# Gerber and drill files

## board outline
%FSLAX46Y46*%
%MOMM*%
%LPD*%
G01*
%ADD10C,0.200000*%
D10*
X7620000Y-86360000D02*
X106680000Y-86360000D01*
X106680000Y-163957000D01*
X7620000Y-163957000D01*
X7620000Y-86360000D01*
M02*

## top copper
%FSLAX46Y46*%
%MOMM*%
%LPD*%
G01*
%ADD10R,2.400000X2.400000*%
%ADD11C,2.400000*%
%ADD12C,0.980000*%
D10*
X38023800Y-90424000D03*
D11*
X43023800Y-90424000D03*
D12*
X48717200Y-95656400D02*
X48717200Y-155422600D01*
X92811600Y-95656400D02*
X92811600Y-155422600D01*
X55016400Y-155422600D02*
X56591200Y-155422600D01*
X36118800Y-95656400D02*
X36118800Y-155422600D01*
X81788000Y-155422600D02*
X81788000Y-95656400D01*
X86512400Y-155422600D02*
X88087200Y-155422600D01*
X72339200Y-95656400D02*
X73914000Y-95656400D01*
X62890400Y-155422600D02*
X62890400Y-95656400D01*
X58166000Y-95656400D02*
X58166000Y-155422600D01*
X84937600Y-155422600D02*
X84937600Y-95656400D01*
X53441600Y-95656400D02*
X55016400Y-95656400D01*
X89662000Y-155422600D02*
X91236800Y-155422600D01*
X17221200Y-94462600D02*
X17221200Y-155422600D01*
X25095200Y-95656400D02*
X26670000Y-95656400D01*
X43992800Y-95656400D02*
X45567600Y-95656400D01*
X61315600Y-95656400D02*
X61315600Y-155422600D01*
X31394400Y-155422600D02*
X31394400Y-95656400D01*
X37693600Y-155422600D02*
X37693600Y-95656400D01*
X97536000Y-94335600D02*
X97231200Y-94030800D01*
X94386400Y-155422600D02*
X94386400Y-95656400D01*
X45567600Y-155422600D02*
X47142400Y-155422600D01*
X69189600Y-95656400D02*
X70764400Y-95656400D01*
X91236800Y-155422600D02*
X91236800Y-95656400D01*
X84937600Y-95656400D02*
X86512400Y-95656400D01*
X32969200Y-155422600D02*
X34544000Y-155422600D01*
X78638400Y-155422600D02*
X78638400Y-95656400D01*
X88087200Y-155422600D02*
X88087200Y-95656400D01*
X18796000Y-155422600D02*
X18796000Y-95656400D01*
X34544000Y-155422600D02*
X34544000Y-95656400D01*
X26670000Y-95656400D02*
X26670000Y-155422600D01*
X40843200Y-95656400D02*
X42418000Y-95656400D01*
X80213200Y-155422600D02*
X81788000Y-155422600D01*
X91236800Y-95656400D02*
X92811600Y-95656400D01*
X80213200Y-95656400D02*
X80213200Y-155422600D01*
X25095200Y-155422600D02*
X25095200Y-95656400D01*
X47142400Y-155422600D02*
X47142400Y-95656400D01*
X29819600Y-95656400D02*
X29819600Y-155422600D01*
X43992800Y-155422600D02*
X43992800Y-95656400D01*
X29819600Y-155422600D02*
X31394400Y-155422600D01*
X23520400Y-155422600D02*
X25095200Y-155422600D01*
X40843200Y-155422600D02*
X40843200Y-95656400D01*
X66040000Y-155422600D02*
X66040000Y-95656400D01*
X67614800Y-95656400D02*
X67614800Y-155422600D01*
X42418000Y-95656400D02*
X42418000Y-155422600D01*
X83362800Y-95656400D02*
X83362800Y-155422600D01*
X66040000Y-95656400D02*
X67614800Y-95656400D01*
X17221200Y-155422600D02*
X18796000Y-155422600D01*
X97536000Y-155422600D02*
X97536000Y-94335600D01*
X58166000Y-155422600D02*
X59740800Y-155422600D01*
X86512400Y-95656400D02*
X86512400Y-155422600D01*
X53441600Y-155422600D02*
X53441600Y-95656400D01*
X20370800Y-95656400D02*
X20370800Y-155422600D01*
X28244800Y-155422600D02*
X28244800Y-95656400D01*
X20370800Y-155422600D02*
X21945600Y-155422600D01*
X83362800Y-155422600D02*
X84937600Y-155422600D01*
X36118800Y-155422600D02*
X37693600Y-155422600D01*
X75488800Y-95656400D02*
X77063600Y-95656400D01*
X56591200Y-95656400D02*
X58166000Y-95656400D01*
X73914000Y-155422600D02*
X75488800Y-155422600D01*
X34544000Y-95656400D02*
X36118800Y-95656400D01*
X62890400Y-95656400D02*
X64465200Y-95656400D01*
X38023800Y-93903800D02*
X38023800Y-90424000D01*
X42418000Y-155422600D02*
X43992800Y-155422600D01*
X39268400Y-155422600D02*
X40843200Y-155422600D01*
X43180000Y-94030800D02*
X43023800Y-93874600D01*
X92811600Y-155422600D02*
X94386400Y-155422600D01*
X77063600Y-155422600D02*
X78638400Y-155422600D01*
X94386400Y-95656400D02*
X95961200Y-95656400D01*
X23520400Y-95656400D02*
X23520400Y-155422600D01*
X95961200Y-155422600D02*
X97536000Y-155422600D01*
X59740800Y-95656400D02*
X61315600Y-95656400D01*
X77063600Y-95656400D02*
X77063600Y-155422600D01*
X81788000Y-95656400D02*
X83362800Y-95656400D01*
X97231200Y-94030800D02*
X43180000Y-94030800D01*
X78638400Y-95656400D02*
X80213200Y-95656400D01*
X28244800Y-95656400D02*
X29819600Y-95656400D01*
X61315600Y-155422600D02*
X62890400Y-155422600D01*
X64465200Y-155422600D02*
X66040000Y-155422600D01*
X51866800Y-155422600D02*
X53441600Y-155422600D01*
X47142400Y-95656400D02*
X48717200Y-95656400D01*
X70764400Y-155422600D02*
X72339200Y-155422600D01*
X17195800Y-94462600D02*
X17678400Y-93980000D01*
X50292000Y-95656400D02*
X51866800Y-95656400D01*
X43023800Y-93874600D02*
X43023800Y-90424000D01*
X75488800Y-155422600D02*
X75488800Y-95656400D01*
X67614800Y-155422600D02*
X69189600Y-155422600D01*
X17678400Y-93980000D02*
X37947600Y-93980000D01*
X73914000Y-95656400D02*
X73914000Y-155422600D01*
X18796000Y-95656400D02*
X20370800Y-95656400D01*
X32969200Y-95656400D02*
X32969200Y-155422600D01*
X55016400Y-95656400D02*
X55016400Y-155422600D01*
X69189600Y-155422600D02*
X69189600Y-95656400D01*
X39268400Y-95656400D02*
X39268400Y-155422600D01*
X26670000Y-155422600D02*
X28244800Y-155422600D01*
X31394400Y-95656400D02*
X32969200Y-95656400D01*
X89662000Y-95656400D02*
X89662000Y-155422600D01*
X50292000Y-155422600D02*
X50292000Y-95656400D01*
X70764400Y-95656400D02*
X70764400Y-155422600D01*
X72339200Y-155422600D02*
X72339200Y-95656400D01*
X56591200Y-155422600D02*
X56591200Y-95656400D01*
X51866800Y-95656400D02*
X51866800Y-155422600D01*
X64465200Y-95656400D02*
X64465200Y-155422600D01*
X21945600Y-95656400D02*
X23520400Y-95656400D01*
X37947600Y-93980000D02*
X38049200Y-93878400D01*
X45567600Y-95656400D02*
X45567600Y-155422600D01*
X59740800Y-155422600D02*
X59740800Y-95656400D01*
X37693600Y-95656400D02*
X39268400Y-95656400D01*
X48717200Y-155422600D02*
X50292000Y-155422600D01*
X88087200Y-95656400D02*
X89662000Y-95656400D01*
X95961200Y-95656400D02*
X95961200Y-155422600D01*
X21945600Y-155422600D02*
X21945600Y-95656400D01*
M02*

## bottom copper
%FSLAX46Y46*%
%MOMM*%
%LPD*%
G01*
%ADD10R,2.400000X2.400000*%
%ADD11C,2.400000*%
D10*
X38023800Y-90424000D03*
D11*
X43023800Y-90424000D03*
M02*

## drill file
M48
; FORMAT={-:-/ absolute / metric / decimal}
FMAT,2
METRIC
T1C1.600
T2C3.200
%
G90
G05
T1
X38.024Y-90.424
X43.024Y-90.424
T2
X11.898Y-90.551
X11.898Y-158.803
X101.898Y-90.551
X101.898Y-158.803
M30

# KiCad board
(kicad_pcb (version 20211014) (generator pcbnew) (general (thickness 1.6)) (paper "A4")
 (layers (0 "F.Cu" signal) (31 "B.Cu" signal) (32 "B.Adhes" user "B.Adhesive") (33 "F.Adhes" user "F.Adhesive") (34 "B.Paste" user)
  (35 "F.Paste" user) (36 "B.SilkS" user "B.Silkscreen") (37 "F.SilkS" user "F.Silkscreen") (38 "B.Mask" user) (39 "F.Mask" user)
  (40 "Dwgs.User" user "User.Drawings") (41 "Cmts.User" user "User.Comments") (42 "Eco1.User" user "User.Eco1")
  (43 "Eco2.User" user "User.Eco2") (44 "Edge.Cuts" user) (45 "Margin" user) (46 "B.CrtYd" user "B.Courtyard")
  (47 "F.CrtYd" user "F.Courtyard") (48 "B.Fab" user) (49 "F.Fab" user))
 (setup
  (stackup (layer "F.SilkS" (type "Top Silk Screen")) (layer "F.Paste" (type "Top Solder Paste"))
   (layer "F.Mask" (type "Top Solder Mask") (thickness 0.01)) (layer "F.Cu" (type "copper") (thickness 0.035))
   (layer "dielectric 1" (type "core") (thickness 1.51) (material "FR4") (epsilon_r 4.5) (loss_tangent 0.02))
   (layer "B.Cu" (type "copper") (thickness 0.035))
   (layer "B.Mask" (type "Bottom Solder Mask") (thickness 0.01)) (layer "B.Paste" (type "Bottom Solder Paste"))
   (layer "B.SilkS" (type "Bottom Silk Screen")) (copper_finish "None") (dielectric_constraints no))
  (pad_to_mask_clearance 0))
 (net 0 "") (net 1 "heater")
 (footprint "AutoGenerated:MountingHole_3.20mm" (layer "F.Cu") (at 91.898 142.803)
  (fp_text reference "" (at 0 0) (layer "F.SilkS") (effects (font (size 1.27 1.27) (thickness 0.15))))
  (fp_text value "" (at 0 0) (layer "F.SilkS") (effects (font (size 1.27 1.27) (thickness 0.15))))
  (pad "" np_thru_hole circle (at 10 16) (size 3.2 3.2) (drill 3.2) (layers F&B.Cu *.Mask)))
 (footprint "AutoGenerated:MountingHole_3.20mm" (layer "F.Cu") (at 11.898 90.551)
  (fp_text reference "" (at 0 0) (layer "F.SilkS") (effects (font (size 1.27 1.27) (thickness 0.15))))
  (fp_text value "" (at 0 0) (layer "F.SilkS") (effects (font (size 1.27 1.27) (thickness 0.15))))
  (pad "" np_thru_hole circle locked (at 0 0) (size 3.2 3.2) (drill 3.2) (layers *.Cu *.Mask)))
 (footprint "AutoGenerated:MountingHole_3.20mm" (layer "F.Cu") (at 91.898 90.551)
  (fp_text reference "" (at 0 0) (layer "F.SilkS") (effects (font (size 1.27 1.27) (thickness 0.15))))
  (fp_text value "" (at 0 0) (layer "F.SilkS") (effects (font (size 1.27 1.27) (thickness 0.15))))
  (pad "" np_thru_hole circle (at 10 0) (size 3.2 3.2) (drill 3.2) (layers F&B.Cu *.Mask)))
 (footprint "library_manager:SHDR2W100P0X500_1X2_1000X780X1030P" (layer "F.Cu") (at 38.0238 90.424)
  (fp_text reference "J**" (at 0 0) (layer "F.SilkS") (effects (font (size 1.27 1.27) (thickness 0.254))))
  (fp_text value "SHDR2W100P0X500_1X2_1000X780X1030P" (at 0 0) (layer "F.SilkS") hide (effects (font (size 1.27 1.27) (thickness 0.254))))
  (pad "1" thru_hole rect locked (at 0 0) (size 2.4 2.4) (drill 1.6) (layers *.Cu *.Mask) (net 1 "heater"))
  (pad "2" thru_hole circle locked (at 5 0) (size 2.4 2.4) (drill 1.6) (layers *.Cu *.Mask) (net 1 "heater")))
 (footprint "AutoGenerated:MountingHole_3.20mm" (layer "F.Cu") (at 11.898 142.803)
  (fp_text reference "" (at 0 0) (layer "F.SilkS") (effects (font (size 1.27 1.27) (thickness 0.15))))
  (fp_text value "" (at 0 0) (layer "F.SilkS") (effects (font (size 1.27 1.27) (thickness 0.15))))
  (pad "" np_thru_hole circle (at 0 16) (size 3.2 3.2) (drill 3.2) (layers F&B.Cu *.Mask)))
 (gr_rect (start 7.62 86.36) (end 106.68 163.957) (layer "Edge.Cuts") (width 0.2) (fill none))
 (segment (start 48.7172 95.6564) (end 48.7172 155.4226) (width 0.98) (layer "F.Cu") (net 1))
 (segment (start 92.8116 95.6564) (end 92.8116 155.4226) (width 0.98) (layer "F.Cu") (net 1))
 (segment (start 55.0164 155.4226) (end 56.5912 155.4226) (width 0.98) (layer "F.Cu") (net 1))
 (segment (start 36.1188 95.6564) (end 36.1188 155.4226) (width 0.98) (layer "F.Cu") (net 1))
 (segment (start 81.788 155.4226) (end 81.788 95.6564) (width 0.98) (layer "F.Cu") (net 1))
 (segment (start 86.5124 155.4226) (end 88.0872 155.4226) (width 0.98) (layer "F.Cu") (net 1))
 (segment (start 72.3392 95.6564) (end 73.914 95.6564) (width 0.98) (layer "F.Cu") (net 1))
 (segment (start 62.8904 155.4226) (end 62.8904 95.6564) (width 0.98) (layer "F.Cu") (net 1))
 (segment (start 58.166 95.6564) (end 58.166 155.4226) (width 0.98) (layer "F.Cu") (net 1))
 (segment (start 84.9376 155.4226) (end 84.9376 95.6564) (width 0.98) (layer "F.Cu") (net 1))
 (segment (start 53.4416 95.6564) (end 55.0164 95.6564) (width 0.98) (layer "F.Cu") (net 1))
 (segment (start 89.662 155.4226) (end 91.2368 155.4226) (width 0.98) (layer "F.Cu") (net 1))
 (segment (start 17.2212 94.4626) (end 17.2212 155.4226) (width 0.98) (layer "F.Cu") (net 1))
 (segment (start 25.0952 95.6564) (end 26.67 95.6564) (width 0.98) (layer "F.Cu") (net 1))
 (segment (start 43.9928 95.6564) (end 45.5676 95.6564) (width 0.98) (layer "F.Cu") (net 1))
 (segment (start 61.3156 95.6564) (end 61.3156 155.4226) (width 0.98) (layer "F.Cu") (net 1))
 (segment (start 31.3944 155.4226) (end 31.3944 95.6564) (width 0.98) (layer "F.Cu") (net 1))
 (segment (start 37.6936 155.4226) (end 37.6936 95.6564) (width 0.98) (layer "F.Cu") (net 1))
 (segment (start 97.536 94.3356) (end 97.2312 94.0308) (width 0.98) (layer "F.Cu") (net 1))
 (segment (start 94.3864 155.4226) (end 94.3864 95.6564) (width 0.98) (layer "F.Cu") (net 1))
 (segment (start 45.5676 155.4226) (end 47.1424 155.4226) (width 0.98) (layer "F.Cu") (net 1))
 (segment (start 69.1896 95.6564) (end 70.7644 95.6564) (width 0.98) (layer "F.Cu") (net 1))
 (segment (start 91.2368 155.4226) (end 91.2368 95.6564) (width 0.98) (layer "F.Cu") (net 1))
 (segment (start 84.9376 95.6564) (end 86.5124 95.6564) (width 0.98) (layer "F.Cu") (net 1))
 (segment (start 32.9692 155.4226) (end 34.544 155.4226) (width 0.98) (layer "F.Cu") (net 1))
 (segment (start 78.6384 155.4226) (end 78.6384 95.6564) (width 0.98) (layer "F.Cu") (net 1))
 (segment (start 88.0872 155.4226) (end 88.0872 95.6564) (width 0.98) (layer "F.Cu") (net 1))
 (segment (start 18.796 155.4226) (end 18.796 95.6564) (width 0.98) (layer "F.Cu") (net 1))
 (segment (start 34.544 155.4226) (end 34.544 95.6564) (width 0.98) (layer "F.Cu") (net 1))
 (segment (start 26.67 95.6564) (end 26.67 155.4226) (width 0.98) (layer "F.Cu") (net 1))
 (segment (start 40.8432 95.6564) (end 42.418 95.6564) (width 0.98) (layer "F.Cu") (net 1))
 (segment (start 80.2132 155.4226) (end 81.788 155.4226) (width 0.98) (layer "F.Cu") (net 1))
 (segment (start 91.2368 95.6564) (end 92.8116 95.6564) (width 0.98) (layer "F.Cu") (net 1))
 (segment (start 80.2132 95.6564) (end 80.2132 155.4226) (width 0.98) (layer "F.Cu") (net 1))
 (segment (start 25.0952 155.4226) (end 25.0952 95.6564) (width 0.98) (layer "F.Cu") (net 1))
 (segment (start 47.1424 155.4226) (end 47.1424 95.6564) (width 0.98) (layer "F.Cu") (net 1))
 (segment (start 29.8196 95.6564) (end 29.8196 155.4226) (width 0.98) (layer "F.Cu") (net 1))
 (segment (start 43.9928 155.4226) (end 43.9928 95.6564) (width 0.98) (layer "F.Cu") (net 1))
 (segment (start 29.8196 155.4226) (end 31.3944 155.4226) (width 0.98) (layer "F.Cu") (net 1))
 (segment (start 23.5204 155.4226) (end 25.0952 155.4226) (width 0.98) (layer "F.Cu") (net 1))
 (segment (start 40.8432 155.4226) (end 40.8432 95.6564) (width 0.98) (layer "F.Cu") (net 1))
 (segment (start 66.04 155.4226) (end 66.04 95.6564) (width 0.98) (layer "F.Cu") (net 1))
 (segment (start 67.6148 95.6564) (end 67.6148 155.4226) (width 0.98) (layer "F.Cu") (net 1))
 (segment (start 42.418 95.6564) (end 42.418 155.4226) (width 0.98) (layer "F.Cu") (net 1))
 (segment (start 83.3628 95.6564) (end 83.3628 155.4226) (width 0.98) (layer "F.Cu") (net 1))
 (segment (start 66.04 95.6564) (end 67.6148 95.6564) (width 0.98) (layer "F.Cu") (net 1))
 (segment (start 17.2212 155.4226) (end 18.796 155.4226) (width 0.98) (layer "F.Cu") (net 1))
 (segment (start 97.536 155.4226) (end 97.536 94.3356) (width 0.98) (layer "F.Cu") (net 1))
 (segment (start 58.166 155.4226) (end 59.7408 155.4226) (width 0.98) (layer "F.Cu") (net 1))
 (segment (start 86.5124 95.6564) (end 86.5124 155.4226) (width 0.98) (layer "F.Cu") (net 1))
 (segment (start 53.4416 155.4226) (end 53.4416 95.6564) (width 0.98) (layer "F.Cu") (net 1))
 (segment (start 20.3708 95.6564) (end 20.3708 155.4226) (width 0.98) (layer "F.Cu") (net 1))
 (segment (start 28.2448 155.4226) (end 28.2448 95.6564) (width 0.98) (layer "F.Cu") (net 1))
 (segment (start 20.3708 155.4226) (end 21.9456 155.4226) (width 0.98) (layer "F.Cu") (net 1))
 (segment (start 83.3628 155.4226) (end 84.9376 155.4226) (width 0.98) (layer "F.Cu") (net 1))
 (segment (start 36.1188 155.4226) (end 37.6936 155.4226) (width 0.98) (layer "F.Cu") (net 1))
 (segment (start 75.4888 95.6564) (end 77.0636 95.6564) (width 0.98) (layer "F.Cu") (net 1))
 (segment (start 56.5912 95.6564) (end 58.166 95.6564) (width 0.98) (layer "F.Cu") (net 1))
 (segment (start 73.914 155.4226) (end 75.4888 155.4226) (width 0.98) (layer "F.Cu") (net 1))
 (segment (start 34.544 95.6564) (end 36.1188 95.6564) (width 0.98) (layer "F.Cu") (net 1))
 (segment (start 62.8904 95.6564) (end 64.4652 95.6564) (width 0.98) (layer "F.Cu") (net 1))
 (segment (start 38.0238 93.9038) (end 38.0238 90.424) (width 0.98) (layer "F.Cu") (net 1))
 (segment (start 42.418 155.4226) (end 43.9928 155.4226) (width 0.98) (layer "F.Cu") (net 1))
 (segment (start 39.2684 155.4226) (end 40.8432 155.4226) (width 0.98) (layer "F.Cu") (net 1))
 (segment (start 43.18 94.0308) (end 43.0238 93.8746) (width 0.98) (layer "F.Cu") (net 1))
 (segment (start 92.8116 155.4226) (end 94.3864 155.4226) (width 0.98) (layer "F.Cu") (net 1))
 (segment (start 77.0636 155.4226) (end 78.6384 155.4226) (width 0.98) (layer "F.Cu") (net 1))
 (segment (start 94.3864 95.6564) (end 95.9612 95.6564) (width 0.98) (layer "F.Cu") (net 1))
 (segment (start 23.5204 95.6564) (end 23.5204 155.4226) (width 0.98) (layer "F.Cu") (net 1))
 (segment (start 95.9612 155.4226) (end 97.536 155.4226) (width 0.98) (layer "F.Cu") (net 1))
 (segment (start 59.7408 95.6564) (end 61.3156 95.6564) (width 0.98) (layer "F.Cu") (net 1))
 (segment (start 77.0636 95.6564) (end 77.0636 155.4226) (width 0.98) (layer "F.Cu") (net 1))
 (segment (start 81.788 95.6564) (end 83.3628 95.6564) (width 0.98) (layer "F.Cu") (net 1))
 (segment (start 97.2312 94.0308) (end 43.18 94.0308) (width 0.98) (layer "F.Cu") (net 1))
 (segment (start 78.6384 95.6564) (end 80.2132 95.6564) (width 0.98) (layer "F.Cu") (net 1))
 (segment (start 28.2448 95.6564) (end 29.8196 95.6564) (width 0.98) (layer "F.Cu") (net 1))
 (segment (start 61.3156 155.4226) (end 62.8904 155.4226) (width 0.98) (layer "F.Cu") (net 1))
 (segment (start 64.4652 155.4226) (end 66.04 155.4226) (width 0.98) (layer "F.Cu") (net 1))
 (segment (start 51.8668 155.4226) (end 53.4416 155.4226) (width 0.98) (layer "F.Cu") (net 1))
 (segment (start 47.1424 95.6564) (end 48.7172 95.6564) (width 0.98) (layer "F.Cu") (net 1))
 (segment (start 70.7644 155.4226) (end 72.3392 155.4226) (width 0.98) (layer "F.Cu") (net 1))
 (segment (start 17.1958 94.4626) (end 17.6784 93.98) (width 0.98) (layer "F.Cu") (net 1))
 (segment (start 50.292 95.6564) (end 51.8668 95.6564) (width 0.98) (layer "F.Cu") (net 1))
 (segment (start 43.0238 93.8746) (end 43.0238 90.424) (width 0.98) (layer "F.Cu") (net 1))
 (segment (start 75.4888 155.4226) (end 75.4888 95.6564) (width 0.98) (layer "F.Cu") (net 1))
 (segment (start 67.6148 155.4226) (end 69.1896 155.4226) (width 0.98) (layer "F.Cu") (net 1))
 (segment (start 17.6784 93.98) (end 37.9476 93.98) (width 0.98) (layer "F.Cu") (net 1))
 (segment (start 73.914 95.6564) (end 73.914 155.4226) (width 0.98) (layer "F.Cu") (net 1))
 (segment (start 18.796 95.6564) (end 20.3708 95.6564) (width 0.98) (layer "F.Cu") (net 1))
 (segment (start 32.9692 95.6564) (end 32.9692 155.4226) (width 0.98) (layer "F.Cu") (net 1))
 (segment (start 55.0164 95.6564) (end 55.0164 155.4226) (width 0.98) (layer "F.Cu") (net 1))
 (segment (start 69.1896 155.4226) (end 69.1896 95.6564) (width 0.98) (layer "F.Cu") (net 1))
 (segment (start 39.2684 95.6564) (end 39.2684 155.4226) (width 0.98) (layer "F.Cu") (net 1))
 (segment (start 26.67 155.4226) (end 28.2448 155.4226) (width 0.98) (layer "F.Cu") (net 1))
 (segment (start 31.3944 95.6564) (end 32.9692 95.6564) (width 0.98) (layer "F.Cu") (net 1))
 (segment (start 89.662 95.6564) (end 89.662 155.4226) (width 0.98) (layer "F.Cu") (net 1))
 (segment (start 50.292 155.4226) (end 50.292 95.6564) (width 0.98) (layer "F.Cu") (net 1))
 (segment (start 70.7644 95.6564) (end 70.7644 155.4226) (width 0.98) (layer "F.Cu") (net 1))
 (segment (start 72.3392 155.4226) (end 72.3392 95.6564) (width 0.98) (layer "F.Cu") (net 1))
 (segment (start 56.5912 155.4226) (end 56.5912 95.6564) (width 0.98) (layer "F.Cu") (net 1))
 (segment (start 51.8668 95.6564) (end 51.8668 155.4226) (width 0.98) (layer "F.Cu") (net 1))
 (segment (start 64.4652 95.6564) (end 64.4652 155.4226) (width 0.98) (layer "F.Cu") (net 1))
 (segment (start 21.9456 95.6564) (end 23.5204 95.6564) (width 0.98) (layer "F.Cu") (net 1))
 (segment (start 37.9476 93.98) (end 38.0492 93.8784) (width 0.98) (layer "F.Cu") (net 1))
 (segment (start 45.5676 95.6564) (end 45.5676 155.4226) (width 0.98) (layer "F.Cu") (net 1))
 (segment (start 59.7408 155.4226) (end 59.7408 95.6564) (width 0.98) (layer "F.Cu") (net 1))
 (segment (start 37.6936 95.6564) (end 39.2684 95.6564) (width 0.98) (layer "F.Cu") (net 1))
 (segment (start 48.7172 155.4226) (end 50.292 155.4226) (width 0.98) (layer "F.Cu") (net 1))
 (segment (start 88.0872 95.6564) (end 89.662 95.6564) (width 0.98) (layer "F.Cu") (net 1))
 (segment (start 95.9612 95.6564) (end 95.9612 155.4226) (width 0.98) (layer "F.Cu") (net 1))
 (segment (start 21.9456 155.4226) (end 21.9456 95.6564) (width 0.98) (layer "F.Cu") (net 1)))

